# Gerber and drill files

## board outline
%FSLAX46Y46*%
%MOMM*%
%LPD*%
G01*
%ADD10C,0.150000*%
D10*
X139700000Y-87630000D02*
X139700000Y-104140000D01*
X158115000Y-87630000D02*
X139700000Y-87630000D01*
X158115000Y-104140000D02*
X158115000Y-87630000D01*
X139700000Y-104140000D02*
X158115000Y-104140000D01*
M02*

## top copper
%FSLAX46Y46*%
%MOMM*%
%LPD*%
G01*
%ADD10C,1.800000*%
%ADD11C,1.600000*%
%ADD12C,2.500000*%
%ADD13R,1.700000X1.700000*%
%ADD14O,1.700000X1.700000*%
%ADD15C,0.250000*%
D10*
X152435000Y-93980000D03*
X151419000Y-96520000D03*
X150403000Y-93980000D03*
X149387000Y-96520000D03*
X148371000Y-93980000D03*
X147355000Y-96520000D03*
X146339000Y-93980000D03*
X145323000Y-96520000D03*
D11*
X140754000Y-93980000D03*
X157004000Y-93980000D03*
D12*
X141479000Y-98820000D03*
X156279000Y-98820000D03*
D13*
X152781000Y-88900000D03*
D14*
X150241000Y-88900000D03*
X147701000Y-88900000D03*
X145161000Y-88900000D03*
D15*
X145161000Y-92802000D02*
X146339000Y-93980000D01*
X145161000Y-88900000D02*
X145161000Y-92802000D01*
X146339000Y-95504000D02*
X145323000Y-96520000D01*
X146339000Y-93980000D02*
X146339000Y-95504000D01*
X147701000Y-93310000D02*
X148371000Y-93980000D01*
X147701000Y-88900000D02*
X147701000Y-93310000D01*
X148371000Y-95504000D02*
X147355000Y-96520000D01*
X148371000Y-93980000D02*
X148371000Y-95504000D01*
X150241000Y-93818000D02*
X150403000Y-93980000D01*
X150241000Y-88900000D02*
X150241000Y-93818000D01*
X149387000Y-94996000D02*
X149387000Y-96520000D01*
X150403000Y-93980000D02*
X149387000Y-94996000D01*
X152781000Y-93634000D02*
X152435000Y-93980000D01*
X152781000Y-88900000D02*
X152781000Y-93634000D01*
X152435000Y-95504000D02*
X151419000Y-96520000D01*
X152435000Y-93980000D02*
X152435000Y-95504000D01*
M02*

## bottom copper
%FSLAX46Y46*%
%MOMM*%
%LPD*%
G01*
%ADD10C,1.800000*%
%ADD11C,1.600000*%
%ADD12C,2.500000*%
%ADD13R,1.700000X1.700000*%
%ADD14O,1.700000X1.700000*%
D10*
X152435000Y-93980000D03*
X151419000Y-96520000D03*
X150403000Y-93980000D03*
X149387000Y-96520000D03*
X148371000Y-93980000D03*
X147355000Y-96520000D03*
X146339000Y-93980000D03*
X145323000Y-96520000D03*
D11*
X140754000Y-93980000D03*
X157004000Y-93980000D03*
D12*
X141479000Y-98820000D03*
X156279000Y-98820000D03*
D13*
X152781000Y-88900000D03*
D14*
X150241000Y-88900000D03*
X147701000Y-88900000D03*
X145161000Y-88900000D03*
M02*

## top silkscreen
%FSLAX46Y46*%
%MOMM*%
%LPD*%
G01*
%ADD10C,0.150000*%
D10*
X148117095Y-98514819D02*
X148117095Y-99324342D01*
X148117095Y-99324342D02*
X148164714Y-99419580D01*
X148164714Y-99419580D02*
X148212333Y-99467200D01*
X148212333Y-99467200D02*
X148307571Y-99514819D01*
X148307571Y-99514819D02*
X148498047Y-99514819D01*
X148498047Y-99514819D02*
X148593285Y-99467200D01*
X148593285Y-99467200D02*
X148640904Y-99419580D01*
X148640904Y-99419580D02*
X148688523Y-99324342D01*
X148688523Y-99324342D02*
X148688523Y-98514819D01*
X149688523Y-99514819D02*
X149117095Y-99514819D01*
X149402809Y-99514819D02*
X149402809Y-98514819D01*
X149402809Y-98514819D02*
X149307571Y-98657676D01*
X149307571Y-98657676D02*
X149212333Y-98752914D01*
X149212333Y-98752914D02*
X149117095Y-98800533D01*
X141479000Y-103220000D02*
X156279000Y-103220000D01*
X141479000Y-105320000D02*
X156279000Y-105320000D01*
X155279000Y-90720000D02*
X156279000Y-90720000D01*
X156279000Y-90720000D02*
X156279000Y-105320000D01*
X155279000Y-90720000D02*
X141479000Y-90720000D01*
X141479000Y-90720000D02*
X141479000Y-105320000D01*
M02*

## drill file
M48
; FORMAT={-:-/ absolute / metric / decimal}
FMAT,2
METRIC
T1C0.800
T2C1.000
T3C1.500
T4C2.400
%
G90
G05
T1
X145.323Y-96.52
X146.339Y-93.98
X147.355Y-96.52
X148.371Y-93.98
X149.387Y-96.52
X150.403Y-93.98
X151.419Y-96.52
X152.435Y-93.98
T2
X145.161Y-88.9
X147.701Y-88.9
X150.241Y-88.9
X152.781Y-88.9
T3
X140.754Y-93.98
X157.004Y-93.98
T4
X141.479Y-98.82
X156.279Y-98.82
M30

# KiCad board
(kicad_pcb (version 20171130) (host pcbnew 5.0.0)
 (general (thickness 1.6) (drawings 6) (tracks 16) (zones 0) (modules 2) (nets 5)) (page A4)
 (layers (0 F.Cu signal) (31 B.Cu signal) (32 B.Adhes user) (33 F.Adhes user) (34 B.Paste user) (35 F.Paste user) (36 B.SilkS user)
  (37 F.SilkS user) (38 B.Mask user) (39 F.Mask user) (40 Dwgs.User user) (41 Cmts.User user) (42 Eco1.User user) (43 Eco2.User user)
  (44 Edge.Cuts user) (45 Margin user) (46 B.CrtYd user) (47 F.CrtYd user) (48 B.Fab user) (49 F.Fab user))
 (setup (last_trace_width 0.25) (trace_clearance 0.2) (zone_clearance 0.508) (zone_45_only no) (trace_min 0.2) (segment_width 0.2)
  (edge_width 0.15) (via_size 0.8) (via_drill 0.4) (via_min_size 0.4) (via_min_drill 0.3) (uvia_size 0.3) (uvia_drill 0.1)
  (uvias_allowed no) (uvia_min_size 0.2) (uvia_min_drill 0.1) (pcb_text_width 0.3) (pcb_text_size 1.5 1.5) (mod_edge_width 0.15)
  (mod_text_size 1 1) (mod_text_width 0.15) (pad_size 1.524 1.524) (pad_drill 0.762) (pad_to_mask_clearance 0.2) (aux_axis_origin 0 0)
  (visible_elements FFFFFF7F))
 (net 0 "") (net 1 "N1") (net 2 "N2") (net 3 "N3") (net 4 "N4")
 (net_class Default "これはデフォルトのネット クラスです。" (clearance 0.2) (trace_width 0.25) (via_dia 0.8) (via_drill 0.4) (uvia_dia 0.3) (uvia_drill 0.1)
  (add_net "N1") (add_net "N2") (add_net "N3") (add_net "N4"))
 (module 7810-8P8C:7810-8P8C (layer F.Cu) (at 148.879 96.52)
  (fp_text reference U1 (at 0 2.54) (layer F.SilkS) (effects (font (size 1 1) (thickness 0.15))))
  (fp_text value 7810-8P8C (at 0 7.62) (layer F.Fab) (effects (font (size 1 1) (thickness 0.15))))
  (fp_line (start -7.4 6.7) (end 7.4 6.7) (layer F.SilkS) (width 0.15))
  (fp_line (start -7.4 8.8) (end 7.4 8.8) (layer F.SilkS) (width 0.15))
  (fp_line (start 6.4 -5.8) (end 7.4 -5.8) (layer F.SilkS) (width 0.15))
  (fp_line (start 7.4 -5.8) (end 7.4 8.8) (layer F.SilkS) (width 0.15))
  (fp_line (start 6.4 -5.8) (end -7.4 -5.8) (layer F.SilkS) (width 0.15))
  (fp_line (start -7.4 -5.8) (end -7.4 8.8) (layer F.SilkS) (width 0.15))
  (pad 1 thru_hole circle (at 3.556 -2.54) (size 1.8 1.8) (drill 0.8) (layers *.Cu *.Mask) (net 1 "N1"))
  (pad 2 thru_hole circle (at 2.54 0) (size 1.8 1.8) (drill 0.8) (layers *.Cu *.Mask) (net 1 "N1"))
  (pad 3 thru_hole circle (at 1.524 -2.54) (size 1.8 1.8) (drill 0.8) (layers *.Cu *.Mask) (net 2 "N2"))
  (pad 4 thru_hole circle (at 0.508 0) (size 1.8 1.8) (drill 0.8) (layers *.Cu *.Mask) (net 2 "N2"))
  (pad 5 thru_hole circle (at -0.508 -2.54) (size 1.8 1.8) (drill 0.8) (layers *.Cu *.Mask) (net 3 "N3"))
  (pad 6 thru_hole circle (at -1.524 0) (size 1.8 1.8) (drill 0.8) (layers *.Cu *.Mask) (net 3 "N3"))
  (pad 7 thru_hole circle (at -2.54 -2.54) (size 1.8 1.8) (drill 0.8) (layers *.Cu *.Mask) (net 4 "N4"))
  (pad 8 thru_hole circle (at -3.556 0) (size 1.8 1.8) (drill 0.8) (layers *.Cu *.Mask) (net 4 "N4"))
  (pad "" np_thru_hole circle (at -8.125 -2.54) (size 1.6 1.6) (drill 1.5) (layers *.Cu *.Mask))
  (pad "" np_thru_hole circle (at 8.125 -2.54) (size 1.6 1.6) (drill 1.5) (layers *.Cu *.Mask))
  (pad "" np_thru_hole circle (at -7.4 2.3) (size 2.5 2.5) (drill 2.4) (layers *.Cu *.Mask))
  (pad "" np_thru_hole circle (at 7.4 2.3) (size 2.5 2.5) (drill 2.4) (layers *.Cu *.Mask)))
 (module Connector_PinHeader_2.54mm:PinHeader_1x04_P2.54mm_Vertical (layer B.Cu) (at 152.781 88.9 90)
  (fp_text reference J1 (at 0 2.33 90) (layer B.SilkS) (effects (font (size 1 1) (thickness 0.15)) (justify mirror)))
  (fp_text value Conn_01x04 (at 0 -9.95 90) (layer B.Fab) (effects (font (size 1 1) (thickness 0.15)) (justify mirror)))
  (pad 1 thru_hole rect (at 0 0 90) (size 1.7 1.7) (drill 1) (layers *.Cu *.Mask) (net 1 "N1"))
  (pad 2 thru_hole oval (at 0 -2.54 90) (size 1.7 1.7) (drill 1) (layers *.Cu *.Mask) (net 2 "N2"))
  (pad 3 thru_hole oval (at 0 -5.08 90) (size 1.7 1.7) (drill 1) (layers *.Cu *.Mask) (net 3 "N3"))
  (pad 4 thru_hole oval (at 0 -7.62 90) (size 1.7 1.7) (drill 1) (layers *.Cu *.Mask) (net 4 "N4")))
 (gr_line (start 139.7 87.63) (end 139.7 104.14) (layer Edge.Cuts) (width 0.15))
 (gr_line (start 158.115 87.63) (end 139.7 87.63) (layer Edge.Cuts) (width 0.15))
 (gr_line (start 158.115 104.14) (end 158.115 87.63) (layer Edge.Cuts) (width 0.15))
 (gr_line (start 139.7 104.14) (end 158.115 104.14) (layer Edge.Cuts) (width 0.15))
 (segment (start 145.161 92.802) (end 146.339 93.98) (width 0.25) (layer F.Cu) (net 4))
 (segment (start 145.161 88.9) (end 145.161 92.802) (width 0.25) (layer F.Cu) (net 4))
 (segment (start 146.339 95.504) (end 145.323 96.52) (width 0.25) (layer F.Cu) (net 4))
 (segment (start 146.339 93.98) (end 146.339 95.504) (width 0.25) (layer F.Cu) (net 4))
 (segment (start 147.701 93.31) (end 148.371 93.98) (width 0.25) (layer F.Cu) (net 3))
 (segment (start 147.701 88.9) (end 147.701 93.31) (width 0.25) (layer F.Cu) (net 3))
 (segment (start 148.371 95.504) (end 147.355 96.52) (width 0.25) (layer F.Cu) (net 3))
 (segment (start 148.371 93.98) (end 148.371 95.504) (width 0.25) (layer F.Cu) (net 3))
 (segment (start 150.241 93.818) (end 150.403 93.98) (width 0.25) (layer F.Cu) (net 2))
 (segment (start 150.241 88.9) (end 150.241 93.818) (width 0.25) (layer F.Cu) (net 2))
 (segment (start 149.387 94.996) (end 149.387 96.52) (width 0.25) (layer F.Cu) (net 2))
 (segment (start 150.403 93.98) (end 149.387 94.996) (width 0.25) (layer F.Cu) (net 2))
 (segment (start 152.781 93.634) (end 152.435 93.98) (width 0.25) (layer F.Cu) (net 1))
 (segment (start 152.781 88.9) (end 152.781 93.634) (width 0.25) (layer F.Cu) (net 1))
 (segment (start 152.435 95.504) (end 151.419 96.52) (width 0.25) (layer F.Cu) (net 1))
 (segment (start 152.435 93.98) (end 152.435 95.504) (width 0.25) (layer F.Cu) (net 1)))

